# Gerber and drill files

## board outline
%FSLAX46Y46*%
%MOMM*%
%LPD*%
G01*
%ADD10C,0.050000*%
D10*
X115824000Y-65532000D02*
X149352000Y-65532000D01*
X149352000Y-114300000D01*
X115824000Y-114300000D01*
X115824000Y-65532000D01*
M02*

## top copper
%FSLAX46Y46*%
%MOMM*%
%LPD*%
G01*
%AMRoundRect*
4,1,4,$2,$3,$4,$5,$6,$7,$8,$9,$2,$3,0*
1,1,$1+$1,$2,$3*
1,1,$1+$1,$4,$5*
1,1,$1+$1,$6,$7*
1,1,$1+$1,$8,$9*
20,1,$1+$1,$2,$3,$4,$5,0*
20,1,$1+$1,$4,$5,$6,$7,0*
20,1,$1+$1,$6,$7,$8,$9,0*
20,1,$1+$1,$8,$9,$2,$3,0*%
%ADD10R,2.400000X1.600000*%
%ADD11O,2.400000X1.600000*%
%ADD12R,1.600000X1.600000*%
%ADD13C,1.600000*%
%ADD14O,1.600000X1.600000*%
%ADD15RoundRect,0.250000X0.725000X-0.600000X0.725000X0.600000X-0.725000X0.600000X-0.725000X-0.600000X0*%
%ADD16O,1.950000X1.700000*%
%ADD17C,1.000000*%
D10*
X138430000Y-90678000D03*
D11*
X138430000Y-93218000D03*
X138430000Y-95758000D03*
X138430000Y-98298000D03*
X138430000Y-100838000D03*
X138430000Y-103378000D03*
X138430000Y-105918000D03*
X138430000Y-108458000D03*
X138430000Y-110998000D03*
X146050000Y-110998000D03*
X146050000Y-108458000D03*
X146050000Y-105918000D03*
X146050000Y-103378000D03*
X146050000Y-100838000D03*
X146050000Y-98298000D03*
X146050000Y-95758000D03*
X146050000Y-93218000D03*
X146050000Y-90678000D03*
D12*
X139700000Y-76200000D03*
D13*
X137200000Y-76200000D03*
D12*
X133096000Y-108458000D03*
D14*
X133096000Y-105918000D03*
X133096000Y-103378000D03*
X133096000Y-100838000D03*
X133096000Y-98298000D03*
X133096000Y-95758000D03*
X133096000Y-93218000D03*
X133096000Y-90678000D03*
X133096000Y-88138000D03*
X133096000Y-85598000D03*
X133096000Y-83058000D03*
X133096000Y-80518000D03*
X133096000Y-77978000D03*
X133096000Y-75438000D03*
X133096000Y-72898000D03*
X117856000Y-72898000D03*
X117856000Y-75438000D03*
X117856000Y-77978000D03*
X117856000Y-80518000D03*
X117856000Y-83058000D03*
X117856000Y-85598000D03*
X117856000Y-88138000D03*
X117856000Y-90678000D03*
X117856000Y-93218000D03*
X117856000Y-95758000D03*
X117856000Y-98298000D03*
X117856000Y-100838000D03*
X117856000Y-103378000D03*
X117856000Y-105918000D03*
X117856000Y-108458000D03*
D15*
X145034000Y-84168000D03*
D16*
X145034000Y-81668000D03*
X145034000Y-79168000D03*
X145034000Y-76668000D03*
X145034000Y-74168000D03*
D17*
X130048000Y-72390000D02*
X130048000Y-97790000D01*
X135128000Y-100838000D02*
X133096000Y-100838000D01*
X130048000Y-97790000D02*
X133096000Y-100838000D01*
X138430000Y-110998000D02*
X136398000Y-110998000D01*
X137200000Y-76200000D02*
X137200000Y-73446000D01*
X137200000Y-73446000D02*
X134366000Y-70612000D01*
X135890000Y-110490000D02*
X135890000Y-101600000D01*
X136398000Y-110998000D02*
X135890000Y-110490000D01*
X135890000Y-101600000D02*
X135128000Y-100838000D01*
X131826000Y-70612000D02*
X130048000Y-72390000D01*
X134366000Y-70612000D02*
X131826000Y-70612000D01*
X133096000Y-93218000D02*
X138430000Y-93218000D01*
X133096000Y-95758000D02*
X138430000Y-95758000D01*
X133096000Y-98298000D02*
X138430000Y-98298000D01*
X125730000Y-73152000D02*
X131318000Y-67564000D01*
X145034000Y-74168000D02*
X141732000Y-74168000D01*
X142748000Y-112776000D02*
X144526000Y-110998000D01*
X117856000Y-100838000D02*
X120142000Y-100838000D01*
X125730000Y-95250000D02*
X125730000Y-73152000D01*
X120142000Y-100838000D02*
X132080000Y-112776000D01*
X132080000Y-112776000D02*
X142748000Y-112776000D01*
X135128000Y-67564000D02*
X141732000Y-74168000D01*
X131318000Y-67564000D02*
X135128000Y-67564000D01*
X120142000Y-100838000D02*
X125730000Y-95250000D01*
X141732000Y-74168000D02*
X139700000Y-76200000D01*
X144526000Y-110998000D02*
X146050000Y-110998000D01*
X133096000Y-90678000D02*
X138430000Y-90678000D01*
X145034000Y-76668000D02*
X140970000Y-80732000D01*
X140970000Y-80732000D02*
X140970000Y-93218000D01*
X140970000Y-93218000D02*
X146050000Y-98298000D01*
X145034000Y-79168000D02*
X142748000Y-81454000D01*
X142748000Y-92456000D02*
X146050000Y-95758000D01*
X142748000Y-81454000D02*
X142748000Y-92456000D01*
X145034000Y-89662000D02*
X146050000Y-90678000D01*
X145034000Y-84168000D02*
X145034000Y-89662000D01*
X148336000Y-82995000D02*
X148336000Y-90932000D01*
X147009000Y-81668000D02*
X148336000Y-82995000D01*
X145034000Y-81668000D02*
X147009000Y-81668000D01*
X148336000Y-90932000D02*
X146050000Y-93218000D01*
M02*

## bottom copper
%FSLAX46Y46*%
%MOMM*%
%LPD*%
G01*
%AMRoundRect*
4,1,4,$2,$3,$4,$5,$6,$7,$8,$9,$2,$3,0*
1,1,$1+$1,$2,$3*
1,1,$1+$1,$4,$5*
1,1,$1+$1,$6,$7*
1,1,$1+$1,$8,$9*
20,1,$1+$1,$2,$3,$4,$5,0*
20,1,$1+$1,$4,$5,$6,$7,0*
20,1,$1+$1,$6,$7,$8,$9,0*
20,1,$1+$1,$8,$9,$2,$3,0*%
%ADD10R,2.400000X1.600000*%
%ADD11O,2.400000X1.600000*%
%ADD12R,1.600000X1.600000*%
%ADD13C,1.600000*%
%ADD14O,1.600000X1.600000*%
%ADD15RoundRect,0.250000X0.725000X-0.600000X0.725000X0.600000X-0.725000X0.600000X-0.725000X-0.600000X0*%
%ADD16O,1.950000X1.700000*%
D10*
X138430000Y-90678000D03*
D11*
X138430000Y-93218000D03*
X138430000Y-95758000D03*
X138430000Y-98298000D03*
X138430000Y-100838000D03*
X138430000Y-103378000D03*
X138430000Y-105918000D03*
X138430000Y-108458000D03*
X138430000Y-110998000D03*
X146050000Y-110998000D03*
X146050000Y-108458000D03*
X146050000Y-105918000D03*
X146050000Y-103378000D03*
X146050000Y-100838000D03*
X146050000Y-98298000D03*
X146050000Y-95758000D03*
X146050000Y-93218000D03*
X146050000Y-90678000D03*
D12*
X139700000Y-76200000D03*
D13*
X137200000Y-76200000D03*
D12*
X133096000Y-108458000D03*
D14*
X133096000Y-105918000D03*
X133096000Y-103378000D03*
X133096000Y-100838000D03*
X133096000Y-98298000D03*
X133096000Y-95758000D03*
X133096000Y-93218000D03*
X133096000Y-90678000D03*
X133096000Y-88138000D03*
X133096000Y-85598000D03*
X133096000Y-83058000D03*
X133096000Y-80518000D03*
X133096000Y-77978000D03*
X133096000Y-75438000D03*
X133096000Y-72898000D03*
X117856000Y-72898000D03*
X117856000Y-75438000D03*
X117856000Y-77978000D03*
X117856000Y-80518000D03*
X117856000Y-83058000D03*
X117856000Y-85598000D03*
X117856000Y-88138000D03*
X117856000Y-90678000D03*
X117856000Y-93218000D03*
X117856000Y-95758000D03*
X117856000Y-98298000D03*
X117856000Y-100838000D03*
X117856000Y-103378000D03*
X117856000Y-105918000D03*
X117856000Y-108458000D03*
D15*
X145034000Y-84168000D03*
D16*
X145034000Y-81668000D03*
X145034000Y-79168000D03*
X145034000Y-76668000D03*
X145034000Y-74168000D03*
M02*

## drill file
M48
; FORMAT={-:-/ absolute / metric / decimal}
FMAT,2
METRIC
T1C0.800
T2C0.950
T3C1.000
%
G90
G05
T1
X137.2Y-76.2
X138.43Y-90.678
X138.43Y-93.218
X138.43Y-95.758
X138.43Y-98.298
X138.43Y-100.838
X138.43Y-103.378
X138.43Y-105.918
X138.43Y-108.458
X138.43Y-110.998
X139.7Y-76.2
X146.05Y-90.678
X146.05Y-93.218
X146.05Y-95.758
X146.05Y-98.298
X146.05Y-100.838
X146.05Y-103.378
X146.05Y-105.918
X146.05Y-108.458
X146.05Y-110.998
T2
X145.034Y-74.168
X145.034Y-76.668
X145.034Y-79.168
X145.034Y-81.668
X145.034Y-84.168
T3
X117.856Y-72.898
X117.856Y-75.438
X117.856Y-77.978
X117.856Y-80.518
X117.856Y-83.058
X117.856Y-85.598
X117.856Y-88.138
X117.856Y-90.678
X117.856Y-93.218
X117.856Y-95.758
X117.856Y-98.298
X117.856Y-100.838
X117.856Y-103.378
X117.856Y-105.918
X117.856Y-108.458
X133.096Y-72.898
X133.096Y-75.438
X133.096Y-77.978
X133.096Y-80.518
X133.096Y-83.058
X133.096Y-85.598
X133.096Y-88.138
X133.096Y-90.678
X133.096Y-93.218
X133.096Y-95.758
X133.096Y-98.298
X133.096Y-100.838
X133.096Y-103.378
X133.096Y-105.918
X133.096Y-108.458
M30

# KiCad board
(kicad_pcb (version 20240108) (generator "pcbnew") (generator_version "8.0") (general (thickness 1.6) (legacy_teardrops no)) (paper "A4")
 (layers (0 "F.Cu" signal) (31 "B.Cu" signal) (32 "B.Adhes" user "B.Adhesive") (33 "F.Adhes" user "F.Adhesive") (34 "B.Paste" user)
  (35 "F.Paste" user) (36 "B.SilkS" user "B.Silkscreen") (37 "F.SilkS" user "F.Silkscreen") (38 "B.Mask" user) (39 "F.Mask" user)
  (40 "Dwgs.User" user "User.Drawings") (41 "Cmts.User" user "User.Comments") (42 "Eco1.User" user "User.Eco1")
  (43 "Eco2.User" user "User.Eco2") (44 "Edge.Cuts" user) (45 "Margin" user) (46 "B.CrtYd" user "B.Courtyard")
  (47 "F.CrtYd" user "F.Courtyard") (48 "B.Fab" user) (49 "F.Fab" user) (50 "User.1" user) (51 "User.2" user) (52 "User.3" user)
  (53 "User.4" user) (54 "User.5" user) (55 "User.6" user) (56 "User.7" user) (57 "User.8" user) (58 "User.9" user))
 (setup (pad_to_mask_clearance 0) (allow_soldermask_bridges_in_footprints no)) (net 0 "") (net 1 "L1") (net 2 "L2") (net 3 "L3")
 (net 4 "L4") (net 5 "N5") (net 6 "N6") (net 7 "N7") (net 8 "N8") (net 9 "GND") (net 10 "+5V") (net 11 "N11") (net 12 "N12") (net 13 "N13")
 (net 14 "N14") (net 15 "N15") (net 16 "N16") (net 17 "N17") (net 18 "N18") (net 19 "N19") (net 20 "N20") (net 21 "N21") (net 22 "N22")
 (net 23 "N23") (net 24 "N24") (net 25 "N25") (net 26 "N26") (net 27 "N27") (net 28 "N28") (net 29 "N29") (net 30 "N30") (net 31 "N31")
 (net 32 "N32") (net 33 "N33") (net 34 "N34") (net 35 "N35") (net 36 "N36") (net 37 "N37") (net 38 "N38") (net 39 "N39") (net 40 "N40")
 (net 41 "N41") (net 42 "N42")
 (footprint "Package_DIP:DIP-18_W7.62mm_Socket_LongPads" (layer "F.Cu") (at 138.43 90.678)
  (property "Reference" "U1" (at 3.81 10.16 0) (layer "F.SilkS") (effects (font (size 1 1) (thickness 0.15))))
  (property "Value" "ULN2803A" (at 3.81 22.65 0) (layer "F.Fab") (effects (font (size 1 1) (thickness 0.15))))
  (pad "1" thru_hole rect (at 0 0) (size 2.4 1.6) (drill 0.8) (layers "*.Cu" "*.Mask") (remove_unused_layers no) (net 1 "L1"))
  (pad "2" thru_hole oval (at 0 2.54) (size 2.4 1.6) (drill 0.8) (layers "*.Cu" "*.Mask") (remove_unused_layers no) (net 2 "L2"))
  (pad "3" thru_hole oval (at 0 5.08) (size 2.4 1.6) (drill 0.8) (layers "*.Cu" "*.Mask") (remove_unused_layers no) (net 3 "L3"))
  (pad "4" thru_hole oval (at 0 7.62) (size 2.4 1.6) (drill 0.8) (layers "*.Cu" "*.Mask") (remove_unused_layers no) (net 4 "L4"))
  (pad "5" thru_hole oval (at 0 10.16) (size 2.4 1.6) (drill 0.8) (layers "*.Cu" "*.Mask") (remove_unused_layers no) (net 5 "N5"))
  (pad "6" thru_hole oval (at 0 12.7) (size 2.4 1.6) (drill 0.8) (layers "*.Cu" "*.Mask") (remove_unused_layers no) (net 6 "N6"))
  (pad "7" thru_hole oval (at 0 15.24) (size 2.4 1.6) (drill 0.8) (layers "*.Cu" "*.Mask") (remove_unused_layers no) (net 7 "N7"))
  (pad "8" thru_hole oval (at 0 17.78) (size 2.4 1.6) (drill 0.8) (layers "*.Cu" "*.Mask") (remove_unused_layers no) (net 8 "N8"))
  (pad "9" thru_hole oval (at 0 20.32) (size 2.4 1.6) (drill 0.8) (layers "*.Cu" "*.Mask") (remove_unused_layers no) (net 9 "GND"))
  (pad "10" thru_hole oval (at 7.62 20.32) (size 2.4 1.6) (drill 0.8) (layers "*.Cu" "*.Mask") (remove_unused_layers no) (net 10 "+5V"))
  (pad "11" thru_hole oval (at 7.62 17.78) (size 2.4 1.6) (drill 0.8) (layers "*.Cu" "*.Mask") (remove_unused_layers no) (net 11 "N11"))
  (pad "12" thru_hole oval (at 7.62 15.24) (size 2.4 1.6) (drill 0.8) (layers "*.Cu" "*.Mask") (remove_unused_layers no) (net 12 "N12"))
  (pad "13" thru_hole oval (at 7.62 12.7) (size 2.4 1.6) (drill 0.8) (layers "*.Cu" "*.Mask") (remove_unused_layers no) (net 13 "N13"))
  (pad "14" thru_hole oval (at 7.62 10.16) (size 2.4 1.6) (drill 0.8) (layers "*.Cu" "*.Mask") (remove_unused_layers no) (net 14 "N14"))
  (pad "15" thru_hole oval (at 7.62 7.62) (size 2.4 1.6) (drill 0.8) (layers "*.Cu" "*.Mask") (remove_unused_layers no) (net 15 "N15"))
  (pad "16" thru_hole oval (at 7.62 5.08) (size 2.4 1.6) (drill 0.8) (layers "*.Cu" "*.Mask") (remove_unused_layers no) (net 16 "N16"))
  (pad "17" thru_hole oval (at 7.62 2.54) (size 2.4 1.6) (drill 0.8) (layers "*.Cu" "*.Mask") (remove_unused_layers no) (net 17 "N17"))
  (pad "18" thru_hole oval (at 7.62 0) (size 2.4 1.6) (drill 0.8) (layers "*.Cu" "*.Mask") (remove_unused_layers no) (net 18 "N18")))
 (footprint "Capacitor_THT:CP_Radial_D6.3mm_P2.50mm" (layer "F.Cu") (at 139.7 76.2 180)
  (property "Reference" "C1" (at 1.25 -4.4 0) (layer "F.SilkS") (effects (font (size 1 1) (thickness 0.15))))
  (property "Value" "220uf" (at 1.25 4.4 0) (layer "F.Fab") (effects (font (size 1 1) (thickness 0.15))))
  (pad "1" thru_hole rect (at 0 0 180) (size 1.6 1.6) (drill 0.8) (layers "*.Cu" "*.Mask") (remove_unused_layers no) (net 10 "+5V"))
  (pad "2" thru_hole circle (at 2.5 0 180) (size 1.6 1.6) (drill 0.8) (layers "*.Cu" "*.Mask") (remove_unused_layers no) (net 9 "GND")))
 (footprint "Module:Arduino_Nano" (layer "F.Cu") (at 133.096 108.458 180)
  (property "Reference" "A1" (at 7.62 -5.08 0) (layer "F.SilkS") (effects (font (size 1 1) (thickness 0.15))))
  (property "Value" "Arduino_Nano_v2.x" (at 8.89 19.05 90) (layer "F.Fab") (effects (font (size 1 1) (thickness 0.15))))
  (pad "1" thru_hole rect (at 0 0 180) (size 1.6 1.6) (drill 1) (layers "*.Cu" "*.Mask") (remove_unused_layers no) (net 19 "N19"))
  (pad "2" thru_hole oval (at 0 2.54 180) (size 1.6 1.6) (drill 1) (layers "*.Cu" "*.Mask") (remove_unused_layers no) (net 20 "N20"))
  (pad "3" thru_hole oval (at 0 5.08 180) (size 1.6 1.6) (drill 1) (layers "*.Cu" "*.Mask") (remove_unused_layers no) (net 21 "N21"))
  (pad "4" thru_hole oval (at 0 7.62 180) (size 1.6 1.6) (drill 1) (layers "*.Cu" "*.Mask") (remove_unused_layers no) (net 9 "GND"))
  (pad "5" thru_hole oval (at 0 10.16 180) (size 1.6 1.6) (drill 1) (layers "*.Cu" "*.Mask") (remove_unused_layers no) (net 4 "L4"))
  (pad "6" thru_hole oval (at 0 12.7 180) (size 1.6 1.6) (drill 1) (layers "*.Cu" "*.Mask") (remove_unused_layers no) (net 3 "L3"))
  (pad "7" thru_hole oval (at 0 15.24 180) (size 1.6 1.6) (drill 1) (layers "*.Cu" "*.Mask") (remove_unused_layers no) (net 2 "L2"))
  (pad "8" thru_hole oval (at 0 17.78 180) (size 1.6 1.6) (drill 1) (layers "*.Cu" "*.Mask") (remove_unused_layers no) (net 1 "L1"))
  (pad "9" thru_hole oval (at 0 20.32 180) (size 1.6 1.6) (drill 1) (layers "*.Cu" "*.Mask") (remove_unused_layers no) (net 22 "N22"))
  (pad "10" thru_hole oval (at 0 22.86 180) (size 1.6 1.6) (drill 1) (layers "*.Cu" "*.Mask") (remove_unused_layers no) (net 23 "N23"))
  (pad "11" thru_hole oval (at 0 25.4 180) (size 1.6 1.6) (drill 1) (layers "*.Cu" "*.Mask") (remove_unused_layers no) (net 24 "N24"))
  (pad "12" thru_hole oval (at 0 27.94 180) (size 1.6 1.6) (drill 1) (layers "*.Cu" "*.Mask") (remove_unused_layers no) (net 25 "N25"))
  (pad "13" thru_hole oval (at 0 30.48 180) (size 1.6 1.6) (drill 1) (layers "*.Cu" "*.Mask") (remove_unused_layers no) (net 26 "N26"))
  (pad "14" thru_hole oval (at 0 33.02 180) (size 1.6 1.6) (drill 1) (layers "*.Cu" "*.Mask") (remove_unused_layers no) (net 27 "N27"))
  (pad "15" thru_hole oval (at 0 35.56 180) (size 1.6 1.6) (drill 1) (layers "*.Cu" "*.Mask") (remove_unused_layers no) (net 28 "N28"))
  (pad "16" thru_hole oval (at 15.24 35.56 180) (size 1.6 1.6) (drill 1) (layers "*.Cu" "*.Mask") (remove_unused_layers no) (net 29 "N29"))
  (pad "17" thru_hole oval (at 15.24 33.02 180) (size 1.6 1.6) (drill 1) (layers "*.Cu" "*.Mask") (remove_unused_layers no) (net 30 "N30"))
  (pad "18" thru_hole oval (at 15.24 30.48 180) (size 1.6 1.6) (drill 1) (layers "*.Cu" "*.Mask") (remove_unused_layers no) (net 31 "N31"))
  (pad "19" thru_hole oval (at 15.24 27.94 180) (size 1.6 1.6) (drill 1) (layers "*.Cu" "*.Mask") (remove_unused_layers no) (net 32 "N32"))
  (pad "20" thru_hole oval (at 15.24 25.4 180) (size 1.6 1.6) (drill 1) (layers "*.Cu" "*.Mask") (remove_unused_layers no) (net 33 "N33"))
  (pad "21" thru_hole oval (at 15.24 22.86 180) (size 1.6 1.6) (drill 1) (layers "*.Cu" "*.Mask") (remove_unused_layers no) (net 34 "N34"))
  (pad "22" thru_hole oval (at 15.24 20.32 180) (size 1.6 1.6) (drill 1) (layers "*.Cu" "*.Mask") (remove_unused_layers no) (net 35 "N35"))
  (pad "23" thru_hole oval (at 15.24 17.78 180) (size 1.6 1.6) (drill 1) (layers "*.Cu" "*.Mask") (remove_unused_layers no) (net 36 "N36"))
  (pad "24" thru_hole oval (at 15.24 15.24 180) (size 1.6 1.6) (drill 1) (layers "*.Cu" "*.Mask") (remove_unused_layers no) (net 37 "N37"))
  (pad "25" thru_hole oval (at 15.24 12.7 180) (size 1.6 1.6) (drill 1) (layers "*.Cu" "*.Mask") (remove_unused_layers no) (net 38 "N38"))
  (pad "26" thru_hole oval (at 15.24 10.16 180) (size 1.6 1.6) (drill 1) (layers "*.Cu" "*.Mask") (remove_unused_layers no) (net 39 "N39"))
  (pad "27" thru_hole oval (at 15.24 7.62 180) (size 1.6 1.6) (drill 1) (layers "*.Cu" "*.Mask") (remove_unused_layers no) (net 10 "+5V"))
  (pad "28" thru_hole oval (at 15.24 5.08 180) (size 1.6 1.6) (drill 1) (layers "*.Cu" "*.Mask") (remove_unused_layers no) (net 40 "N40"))
  (pad "29" thru_hole oval (at 15.24 2.54 180) (size 1.6 1.6) (drill 1) (layers "*.Cu" "*.Mask") (remove_unused_layers no) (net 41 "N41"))
  (pad "30" thru_hole oval (at 15.24 0 180) (size 1.6 1.6) (drill 1) (layers "*.Cu" "*.Mask") (remove_unused_layers no) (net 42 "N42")))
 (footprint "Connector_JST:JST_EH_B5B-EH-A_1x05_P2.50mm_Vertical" (layer "F.Cu") (at 145.034 84.168 90)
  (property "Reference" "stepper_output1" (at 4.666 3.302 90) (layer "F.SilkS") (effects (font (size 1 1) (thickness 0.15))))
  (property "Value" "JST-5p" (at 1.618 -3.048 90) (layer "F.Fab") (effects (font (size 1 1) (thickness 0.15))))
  (pad "1" thru_hole roundrect (at 0 0 90) (size 1.7 1.95) (drill 0.95) (layers "*.Cu" "*.Mask") (remove_unused_layers no)
   (roundrect_rratio 0.147059) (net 18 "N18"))
  (pad "2" thru_hole oval (at 2.5 0 90) (size 1.7 1.95) (drill 0.95) (layers "*.Cu" "*.Mask") (remove_unused_layers no) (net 17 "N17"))
  (pad "3" thru_hole oval (at 5 0 90) (size 1.7 1.95) (drill 0.95) (layers "*.Cu" "*.Mask") (remove_unused_layers no) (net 16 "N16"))
  (pad "4" thru_hole oval (at 7.5 0 90) (size 1.7 1.95) (drill 0.95) (layers "*.Cu" "*.Mask") (remove_unused_layers no) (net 15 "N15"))
  (pad "5" thru_hole oval (at 10 0 90) (size 1.7 1.95) (drill 0.95) (layers "*.Cu" "*.Mask") (remove_unused_layers no) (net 10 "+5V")))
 (gr_rect (start 115.824 65.532) (end 149.352 114.3) (stroke (width 0.05) (type default)) (fill none) (layer "Edge.Cuts"))
 (segment (start 130.048 72.39) (end 130.048 97.79) (width 1) (layer "F.Cu") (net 9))
 (segment (start 135.128 100.838) (end 133.096 100.838) (width 1) (layer "F.Cu") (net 9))
 (segment (start 130.048 97.79) (end 133.096 100.838) (width 1) (layer "F.Cu") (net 9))
 (segment (start 138.43 110.998) (end 136.398 110.998) (width 1) (layer "F.Cu") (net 9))
 (segment (start 137.2 76.2) (end 137.2 73.446) (width 1) (layer "F.Cu") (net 9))
 (segment (start 137.2 73.446) (end 134.366 70.612) (width 1) (layer "F.Cu") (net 9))
 (segment (start 135.89 110.49) (end 135.89 101.6) (width 1) (layer "F.Cu") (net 9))
 (segment (start 136.398 110.998) (end 135.89 110.49) (width 1) (layer "F.Cu") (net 9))
 (segment (start 135.89 101.6) (end 135.128 100.838) (width 1) (layer "F.Cu") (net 9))
 (segment (start 131.826 70.612) (end 130.048 72.39) (width 1) (layer "F.Cu") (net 9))
 (segment (start 134.366 70.612) (end 131.826 70.612) (width 1) (layer "F.Cu") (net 9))
 (segment (start 133.096 93.218) (end 138.43 93.218) (width 1) (layer "F.Cu") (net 2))
 (segment (start 133.096 95.758) (end 138.43 95.758) (width 1) (layer "F.Cu") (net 3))
 (segment (start 133.096 98.298) (end 138.43 98.298) (width 1) (layer "F.Cu") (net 4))
 (segment (start 125.73 73.152) (end 131.318 67.564) (width 1) (layer "F.Cu") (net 10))
 (segment (start 145.034 74.168) (end 141.732 74.168) (width 1) (layer "F.Cu") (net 10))
 (segment (start 142.748 112.776) (end 144.526 110.998) (width 1) (layer "F.Cu") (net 10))
 (segment (start 117.856 100.838) (end 120.142 100.838) (width 1) (layer "F.Cu") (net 10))
 (segment (start 125.73 95.25) (end 125.73 73.152) (width 1) (layer "F.Cu") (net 10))
 (segment (start 120.142 100.838) (end 132.08 112.776) (width 1) (layer "F.Cu") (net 10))
 (segment (start 132.08 112.776) (end 142.748 112.776) (width 1) (layer "F.Cu") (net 10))
 (segment (start 135.128 67.564) (end 141.732 74.168) (width 1) (layer "F.Cu") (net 10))
 (segment (start 131.318 67.564) (end 135.128 67.564) (width 1) (layer "F.Cu") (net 10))
 (segment (start 120.142 100.838) (end 125.73 95.25) (width 1) (layer "F.Cu") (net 10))
 (segment (start 141.732 74.168) (end 139.7 76.2) (width 1) (layer "F.Cu") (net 10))
 (segment (start 144.526 110.998) (end 146.05 110.998) (width 1) (layer "F.Cu") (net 10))
 (segment (start 133.096 90.678) (end 138.43 90.678) (width 1) (layer "F.Cu") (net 1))
 (segment (start 145.034 76.668) (end 140.97 80.732) (width 1) (layer "F.Cu") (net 15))
 (segment (start 140.97 80.732) (end 140.97 93.218) (width 1) (layer "F.Cu") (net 15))
 (segment (start 140.97 93.218) (end 146.05 98.298) (width 1) (layer "F.Cu") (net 15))
 (segment (start 145.034 79.168) (end 142.748 81.454) (width 1) (layer "F.Cu") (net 16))
 (segment (start 142.748 92.456) (end 146.05 95.758) (width 1) (layer "F.Cu") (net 16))
 (segment (start 142.748 81.454) (end 142.748 92.456) (width 1) (layer "F.Cu") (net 16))
 (segment (start 145.034 89.662) (end 146.05 90.678) (width 1) (layer "F.Cu") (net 18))
 (segment (start 145.034 84.168) (end 145.034 89.662) (width 1) (layer "F.Cu") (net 18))
 (segment (start 148.336 82.995) (end 148.336 90.932) (width 1) (layer "F.Cu") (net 17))
 (segment (start 147.009 81.668) (end 148.336 82.995) (width 1) (layer "F.Cu") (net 17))
 (segment (start 145.034 81.668) (end 147.009 81.668) (width 1) (layer "F.Cu") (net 17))
 (segment (start 148.336 90.932) (end 146.05 93.218) (width 1) (layer "F.Cu") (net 17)))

